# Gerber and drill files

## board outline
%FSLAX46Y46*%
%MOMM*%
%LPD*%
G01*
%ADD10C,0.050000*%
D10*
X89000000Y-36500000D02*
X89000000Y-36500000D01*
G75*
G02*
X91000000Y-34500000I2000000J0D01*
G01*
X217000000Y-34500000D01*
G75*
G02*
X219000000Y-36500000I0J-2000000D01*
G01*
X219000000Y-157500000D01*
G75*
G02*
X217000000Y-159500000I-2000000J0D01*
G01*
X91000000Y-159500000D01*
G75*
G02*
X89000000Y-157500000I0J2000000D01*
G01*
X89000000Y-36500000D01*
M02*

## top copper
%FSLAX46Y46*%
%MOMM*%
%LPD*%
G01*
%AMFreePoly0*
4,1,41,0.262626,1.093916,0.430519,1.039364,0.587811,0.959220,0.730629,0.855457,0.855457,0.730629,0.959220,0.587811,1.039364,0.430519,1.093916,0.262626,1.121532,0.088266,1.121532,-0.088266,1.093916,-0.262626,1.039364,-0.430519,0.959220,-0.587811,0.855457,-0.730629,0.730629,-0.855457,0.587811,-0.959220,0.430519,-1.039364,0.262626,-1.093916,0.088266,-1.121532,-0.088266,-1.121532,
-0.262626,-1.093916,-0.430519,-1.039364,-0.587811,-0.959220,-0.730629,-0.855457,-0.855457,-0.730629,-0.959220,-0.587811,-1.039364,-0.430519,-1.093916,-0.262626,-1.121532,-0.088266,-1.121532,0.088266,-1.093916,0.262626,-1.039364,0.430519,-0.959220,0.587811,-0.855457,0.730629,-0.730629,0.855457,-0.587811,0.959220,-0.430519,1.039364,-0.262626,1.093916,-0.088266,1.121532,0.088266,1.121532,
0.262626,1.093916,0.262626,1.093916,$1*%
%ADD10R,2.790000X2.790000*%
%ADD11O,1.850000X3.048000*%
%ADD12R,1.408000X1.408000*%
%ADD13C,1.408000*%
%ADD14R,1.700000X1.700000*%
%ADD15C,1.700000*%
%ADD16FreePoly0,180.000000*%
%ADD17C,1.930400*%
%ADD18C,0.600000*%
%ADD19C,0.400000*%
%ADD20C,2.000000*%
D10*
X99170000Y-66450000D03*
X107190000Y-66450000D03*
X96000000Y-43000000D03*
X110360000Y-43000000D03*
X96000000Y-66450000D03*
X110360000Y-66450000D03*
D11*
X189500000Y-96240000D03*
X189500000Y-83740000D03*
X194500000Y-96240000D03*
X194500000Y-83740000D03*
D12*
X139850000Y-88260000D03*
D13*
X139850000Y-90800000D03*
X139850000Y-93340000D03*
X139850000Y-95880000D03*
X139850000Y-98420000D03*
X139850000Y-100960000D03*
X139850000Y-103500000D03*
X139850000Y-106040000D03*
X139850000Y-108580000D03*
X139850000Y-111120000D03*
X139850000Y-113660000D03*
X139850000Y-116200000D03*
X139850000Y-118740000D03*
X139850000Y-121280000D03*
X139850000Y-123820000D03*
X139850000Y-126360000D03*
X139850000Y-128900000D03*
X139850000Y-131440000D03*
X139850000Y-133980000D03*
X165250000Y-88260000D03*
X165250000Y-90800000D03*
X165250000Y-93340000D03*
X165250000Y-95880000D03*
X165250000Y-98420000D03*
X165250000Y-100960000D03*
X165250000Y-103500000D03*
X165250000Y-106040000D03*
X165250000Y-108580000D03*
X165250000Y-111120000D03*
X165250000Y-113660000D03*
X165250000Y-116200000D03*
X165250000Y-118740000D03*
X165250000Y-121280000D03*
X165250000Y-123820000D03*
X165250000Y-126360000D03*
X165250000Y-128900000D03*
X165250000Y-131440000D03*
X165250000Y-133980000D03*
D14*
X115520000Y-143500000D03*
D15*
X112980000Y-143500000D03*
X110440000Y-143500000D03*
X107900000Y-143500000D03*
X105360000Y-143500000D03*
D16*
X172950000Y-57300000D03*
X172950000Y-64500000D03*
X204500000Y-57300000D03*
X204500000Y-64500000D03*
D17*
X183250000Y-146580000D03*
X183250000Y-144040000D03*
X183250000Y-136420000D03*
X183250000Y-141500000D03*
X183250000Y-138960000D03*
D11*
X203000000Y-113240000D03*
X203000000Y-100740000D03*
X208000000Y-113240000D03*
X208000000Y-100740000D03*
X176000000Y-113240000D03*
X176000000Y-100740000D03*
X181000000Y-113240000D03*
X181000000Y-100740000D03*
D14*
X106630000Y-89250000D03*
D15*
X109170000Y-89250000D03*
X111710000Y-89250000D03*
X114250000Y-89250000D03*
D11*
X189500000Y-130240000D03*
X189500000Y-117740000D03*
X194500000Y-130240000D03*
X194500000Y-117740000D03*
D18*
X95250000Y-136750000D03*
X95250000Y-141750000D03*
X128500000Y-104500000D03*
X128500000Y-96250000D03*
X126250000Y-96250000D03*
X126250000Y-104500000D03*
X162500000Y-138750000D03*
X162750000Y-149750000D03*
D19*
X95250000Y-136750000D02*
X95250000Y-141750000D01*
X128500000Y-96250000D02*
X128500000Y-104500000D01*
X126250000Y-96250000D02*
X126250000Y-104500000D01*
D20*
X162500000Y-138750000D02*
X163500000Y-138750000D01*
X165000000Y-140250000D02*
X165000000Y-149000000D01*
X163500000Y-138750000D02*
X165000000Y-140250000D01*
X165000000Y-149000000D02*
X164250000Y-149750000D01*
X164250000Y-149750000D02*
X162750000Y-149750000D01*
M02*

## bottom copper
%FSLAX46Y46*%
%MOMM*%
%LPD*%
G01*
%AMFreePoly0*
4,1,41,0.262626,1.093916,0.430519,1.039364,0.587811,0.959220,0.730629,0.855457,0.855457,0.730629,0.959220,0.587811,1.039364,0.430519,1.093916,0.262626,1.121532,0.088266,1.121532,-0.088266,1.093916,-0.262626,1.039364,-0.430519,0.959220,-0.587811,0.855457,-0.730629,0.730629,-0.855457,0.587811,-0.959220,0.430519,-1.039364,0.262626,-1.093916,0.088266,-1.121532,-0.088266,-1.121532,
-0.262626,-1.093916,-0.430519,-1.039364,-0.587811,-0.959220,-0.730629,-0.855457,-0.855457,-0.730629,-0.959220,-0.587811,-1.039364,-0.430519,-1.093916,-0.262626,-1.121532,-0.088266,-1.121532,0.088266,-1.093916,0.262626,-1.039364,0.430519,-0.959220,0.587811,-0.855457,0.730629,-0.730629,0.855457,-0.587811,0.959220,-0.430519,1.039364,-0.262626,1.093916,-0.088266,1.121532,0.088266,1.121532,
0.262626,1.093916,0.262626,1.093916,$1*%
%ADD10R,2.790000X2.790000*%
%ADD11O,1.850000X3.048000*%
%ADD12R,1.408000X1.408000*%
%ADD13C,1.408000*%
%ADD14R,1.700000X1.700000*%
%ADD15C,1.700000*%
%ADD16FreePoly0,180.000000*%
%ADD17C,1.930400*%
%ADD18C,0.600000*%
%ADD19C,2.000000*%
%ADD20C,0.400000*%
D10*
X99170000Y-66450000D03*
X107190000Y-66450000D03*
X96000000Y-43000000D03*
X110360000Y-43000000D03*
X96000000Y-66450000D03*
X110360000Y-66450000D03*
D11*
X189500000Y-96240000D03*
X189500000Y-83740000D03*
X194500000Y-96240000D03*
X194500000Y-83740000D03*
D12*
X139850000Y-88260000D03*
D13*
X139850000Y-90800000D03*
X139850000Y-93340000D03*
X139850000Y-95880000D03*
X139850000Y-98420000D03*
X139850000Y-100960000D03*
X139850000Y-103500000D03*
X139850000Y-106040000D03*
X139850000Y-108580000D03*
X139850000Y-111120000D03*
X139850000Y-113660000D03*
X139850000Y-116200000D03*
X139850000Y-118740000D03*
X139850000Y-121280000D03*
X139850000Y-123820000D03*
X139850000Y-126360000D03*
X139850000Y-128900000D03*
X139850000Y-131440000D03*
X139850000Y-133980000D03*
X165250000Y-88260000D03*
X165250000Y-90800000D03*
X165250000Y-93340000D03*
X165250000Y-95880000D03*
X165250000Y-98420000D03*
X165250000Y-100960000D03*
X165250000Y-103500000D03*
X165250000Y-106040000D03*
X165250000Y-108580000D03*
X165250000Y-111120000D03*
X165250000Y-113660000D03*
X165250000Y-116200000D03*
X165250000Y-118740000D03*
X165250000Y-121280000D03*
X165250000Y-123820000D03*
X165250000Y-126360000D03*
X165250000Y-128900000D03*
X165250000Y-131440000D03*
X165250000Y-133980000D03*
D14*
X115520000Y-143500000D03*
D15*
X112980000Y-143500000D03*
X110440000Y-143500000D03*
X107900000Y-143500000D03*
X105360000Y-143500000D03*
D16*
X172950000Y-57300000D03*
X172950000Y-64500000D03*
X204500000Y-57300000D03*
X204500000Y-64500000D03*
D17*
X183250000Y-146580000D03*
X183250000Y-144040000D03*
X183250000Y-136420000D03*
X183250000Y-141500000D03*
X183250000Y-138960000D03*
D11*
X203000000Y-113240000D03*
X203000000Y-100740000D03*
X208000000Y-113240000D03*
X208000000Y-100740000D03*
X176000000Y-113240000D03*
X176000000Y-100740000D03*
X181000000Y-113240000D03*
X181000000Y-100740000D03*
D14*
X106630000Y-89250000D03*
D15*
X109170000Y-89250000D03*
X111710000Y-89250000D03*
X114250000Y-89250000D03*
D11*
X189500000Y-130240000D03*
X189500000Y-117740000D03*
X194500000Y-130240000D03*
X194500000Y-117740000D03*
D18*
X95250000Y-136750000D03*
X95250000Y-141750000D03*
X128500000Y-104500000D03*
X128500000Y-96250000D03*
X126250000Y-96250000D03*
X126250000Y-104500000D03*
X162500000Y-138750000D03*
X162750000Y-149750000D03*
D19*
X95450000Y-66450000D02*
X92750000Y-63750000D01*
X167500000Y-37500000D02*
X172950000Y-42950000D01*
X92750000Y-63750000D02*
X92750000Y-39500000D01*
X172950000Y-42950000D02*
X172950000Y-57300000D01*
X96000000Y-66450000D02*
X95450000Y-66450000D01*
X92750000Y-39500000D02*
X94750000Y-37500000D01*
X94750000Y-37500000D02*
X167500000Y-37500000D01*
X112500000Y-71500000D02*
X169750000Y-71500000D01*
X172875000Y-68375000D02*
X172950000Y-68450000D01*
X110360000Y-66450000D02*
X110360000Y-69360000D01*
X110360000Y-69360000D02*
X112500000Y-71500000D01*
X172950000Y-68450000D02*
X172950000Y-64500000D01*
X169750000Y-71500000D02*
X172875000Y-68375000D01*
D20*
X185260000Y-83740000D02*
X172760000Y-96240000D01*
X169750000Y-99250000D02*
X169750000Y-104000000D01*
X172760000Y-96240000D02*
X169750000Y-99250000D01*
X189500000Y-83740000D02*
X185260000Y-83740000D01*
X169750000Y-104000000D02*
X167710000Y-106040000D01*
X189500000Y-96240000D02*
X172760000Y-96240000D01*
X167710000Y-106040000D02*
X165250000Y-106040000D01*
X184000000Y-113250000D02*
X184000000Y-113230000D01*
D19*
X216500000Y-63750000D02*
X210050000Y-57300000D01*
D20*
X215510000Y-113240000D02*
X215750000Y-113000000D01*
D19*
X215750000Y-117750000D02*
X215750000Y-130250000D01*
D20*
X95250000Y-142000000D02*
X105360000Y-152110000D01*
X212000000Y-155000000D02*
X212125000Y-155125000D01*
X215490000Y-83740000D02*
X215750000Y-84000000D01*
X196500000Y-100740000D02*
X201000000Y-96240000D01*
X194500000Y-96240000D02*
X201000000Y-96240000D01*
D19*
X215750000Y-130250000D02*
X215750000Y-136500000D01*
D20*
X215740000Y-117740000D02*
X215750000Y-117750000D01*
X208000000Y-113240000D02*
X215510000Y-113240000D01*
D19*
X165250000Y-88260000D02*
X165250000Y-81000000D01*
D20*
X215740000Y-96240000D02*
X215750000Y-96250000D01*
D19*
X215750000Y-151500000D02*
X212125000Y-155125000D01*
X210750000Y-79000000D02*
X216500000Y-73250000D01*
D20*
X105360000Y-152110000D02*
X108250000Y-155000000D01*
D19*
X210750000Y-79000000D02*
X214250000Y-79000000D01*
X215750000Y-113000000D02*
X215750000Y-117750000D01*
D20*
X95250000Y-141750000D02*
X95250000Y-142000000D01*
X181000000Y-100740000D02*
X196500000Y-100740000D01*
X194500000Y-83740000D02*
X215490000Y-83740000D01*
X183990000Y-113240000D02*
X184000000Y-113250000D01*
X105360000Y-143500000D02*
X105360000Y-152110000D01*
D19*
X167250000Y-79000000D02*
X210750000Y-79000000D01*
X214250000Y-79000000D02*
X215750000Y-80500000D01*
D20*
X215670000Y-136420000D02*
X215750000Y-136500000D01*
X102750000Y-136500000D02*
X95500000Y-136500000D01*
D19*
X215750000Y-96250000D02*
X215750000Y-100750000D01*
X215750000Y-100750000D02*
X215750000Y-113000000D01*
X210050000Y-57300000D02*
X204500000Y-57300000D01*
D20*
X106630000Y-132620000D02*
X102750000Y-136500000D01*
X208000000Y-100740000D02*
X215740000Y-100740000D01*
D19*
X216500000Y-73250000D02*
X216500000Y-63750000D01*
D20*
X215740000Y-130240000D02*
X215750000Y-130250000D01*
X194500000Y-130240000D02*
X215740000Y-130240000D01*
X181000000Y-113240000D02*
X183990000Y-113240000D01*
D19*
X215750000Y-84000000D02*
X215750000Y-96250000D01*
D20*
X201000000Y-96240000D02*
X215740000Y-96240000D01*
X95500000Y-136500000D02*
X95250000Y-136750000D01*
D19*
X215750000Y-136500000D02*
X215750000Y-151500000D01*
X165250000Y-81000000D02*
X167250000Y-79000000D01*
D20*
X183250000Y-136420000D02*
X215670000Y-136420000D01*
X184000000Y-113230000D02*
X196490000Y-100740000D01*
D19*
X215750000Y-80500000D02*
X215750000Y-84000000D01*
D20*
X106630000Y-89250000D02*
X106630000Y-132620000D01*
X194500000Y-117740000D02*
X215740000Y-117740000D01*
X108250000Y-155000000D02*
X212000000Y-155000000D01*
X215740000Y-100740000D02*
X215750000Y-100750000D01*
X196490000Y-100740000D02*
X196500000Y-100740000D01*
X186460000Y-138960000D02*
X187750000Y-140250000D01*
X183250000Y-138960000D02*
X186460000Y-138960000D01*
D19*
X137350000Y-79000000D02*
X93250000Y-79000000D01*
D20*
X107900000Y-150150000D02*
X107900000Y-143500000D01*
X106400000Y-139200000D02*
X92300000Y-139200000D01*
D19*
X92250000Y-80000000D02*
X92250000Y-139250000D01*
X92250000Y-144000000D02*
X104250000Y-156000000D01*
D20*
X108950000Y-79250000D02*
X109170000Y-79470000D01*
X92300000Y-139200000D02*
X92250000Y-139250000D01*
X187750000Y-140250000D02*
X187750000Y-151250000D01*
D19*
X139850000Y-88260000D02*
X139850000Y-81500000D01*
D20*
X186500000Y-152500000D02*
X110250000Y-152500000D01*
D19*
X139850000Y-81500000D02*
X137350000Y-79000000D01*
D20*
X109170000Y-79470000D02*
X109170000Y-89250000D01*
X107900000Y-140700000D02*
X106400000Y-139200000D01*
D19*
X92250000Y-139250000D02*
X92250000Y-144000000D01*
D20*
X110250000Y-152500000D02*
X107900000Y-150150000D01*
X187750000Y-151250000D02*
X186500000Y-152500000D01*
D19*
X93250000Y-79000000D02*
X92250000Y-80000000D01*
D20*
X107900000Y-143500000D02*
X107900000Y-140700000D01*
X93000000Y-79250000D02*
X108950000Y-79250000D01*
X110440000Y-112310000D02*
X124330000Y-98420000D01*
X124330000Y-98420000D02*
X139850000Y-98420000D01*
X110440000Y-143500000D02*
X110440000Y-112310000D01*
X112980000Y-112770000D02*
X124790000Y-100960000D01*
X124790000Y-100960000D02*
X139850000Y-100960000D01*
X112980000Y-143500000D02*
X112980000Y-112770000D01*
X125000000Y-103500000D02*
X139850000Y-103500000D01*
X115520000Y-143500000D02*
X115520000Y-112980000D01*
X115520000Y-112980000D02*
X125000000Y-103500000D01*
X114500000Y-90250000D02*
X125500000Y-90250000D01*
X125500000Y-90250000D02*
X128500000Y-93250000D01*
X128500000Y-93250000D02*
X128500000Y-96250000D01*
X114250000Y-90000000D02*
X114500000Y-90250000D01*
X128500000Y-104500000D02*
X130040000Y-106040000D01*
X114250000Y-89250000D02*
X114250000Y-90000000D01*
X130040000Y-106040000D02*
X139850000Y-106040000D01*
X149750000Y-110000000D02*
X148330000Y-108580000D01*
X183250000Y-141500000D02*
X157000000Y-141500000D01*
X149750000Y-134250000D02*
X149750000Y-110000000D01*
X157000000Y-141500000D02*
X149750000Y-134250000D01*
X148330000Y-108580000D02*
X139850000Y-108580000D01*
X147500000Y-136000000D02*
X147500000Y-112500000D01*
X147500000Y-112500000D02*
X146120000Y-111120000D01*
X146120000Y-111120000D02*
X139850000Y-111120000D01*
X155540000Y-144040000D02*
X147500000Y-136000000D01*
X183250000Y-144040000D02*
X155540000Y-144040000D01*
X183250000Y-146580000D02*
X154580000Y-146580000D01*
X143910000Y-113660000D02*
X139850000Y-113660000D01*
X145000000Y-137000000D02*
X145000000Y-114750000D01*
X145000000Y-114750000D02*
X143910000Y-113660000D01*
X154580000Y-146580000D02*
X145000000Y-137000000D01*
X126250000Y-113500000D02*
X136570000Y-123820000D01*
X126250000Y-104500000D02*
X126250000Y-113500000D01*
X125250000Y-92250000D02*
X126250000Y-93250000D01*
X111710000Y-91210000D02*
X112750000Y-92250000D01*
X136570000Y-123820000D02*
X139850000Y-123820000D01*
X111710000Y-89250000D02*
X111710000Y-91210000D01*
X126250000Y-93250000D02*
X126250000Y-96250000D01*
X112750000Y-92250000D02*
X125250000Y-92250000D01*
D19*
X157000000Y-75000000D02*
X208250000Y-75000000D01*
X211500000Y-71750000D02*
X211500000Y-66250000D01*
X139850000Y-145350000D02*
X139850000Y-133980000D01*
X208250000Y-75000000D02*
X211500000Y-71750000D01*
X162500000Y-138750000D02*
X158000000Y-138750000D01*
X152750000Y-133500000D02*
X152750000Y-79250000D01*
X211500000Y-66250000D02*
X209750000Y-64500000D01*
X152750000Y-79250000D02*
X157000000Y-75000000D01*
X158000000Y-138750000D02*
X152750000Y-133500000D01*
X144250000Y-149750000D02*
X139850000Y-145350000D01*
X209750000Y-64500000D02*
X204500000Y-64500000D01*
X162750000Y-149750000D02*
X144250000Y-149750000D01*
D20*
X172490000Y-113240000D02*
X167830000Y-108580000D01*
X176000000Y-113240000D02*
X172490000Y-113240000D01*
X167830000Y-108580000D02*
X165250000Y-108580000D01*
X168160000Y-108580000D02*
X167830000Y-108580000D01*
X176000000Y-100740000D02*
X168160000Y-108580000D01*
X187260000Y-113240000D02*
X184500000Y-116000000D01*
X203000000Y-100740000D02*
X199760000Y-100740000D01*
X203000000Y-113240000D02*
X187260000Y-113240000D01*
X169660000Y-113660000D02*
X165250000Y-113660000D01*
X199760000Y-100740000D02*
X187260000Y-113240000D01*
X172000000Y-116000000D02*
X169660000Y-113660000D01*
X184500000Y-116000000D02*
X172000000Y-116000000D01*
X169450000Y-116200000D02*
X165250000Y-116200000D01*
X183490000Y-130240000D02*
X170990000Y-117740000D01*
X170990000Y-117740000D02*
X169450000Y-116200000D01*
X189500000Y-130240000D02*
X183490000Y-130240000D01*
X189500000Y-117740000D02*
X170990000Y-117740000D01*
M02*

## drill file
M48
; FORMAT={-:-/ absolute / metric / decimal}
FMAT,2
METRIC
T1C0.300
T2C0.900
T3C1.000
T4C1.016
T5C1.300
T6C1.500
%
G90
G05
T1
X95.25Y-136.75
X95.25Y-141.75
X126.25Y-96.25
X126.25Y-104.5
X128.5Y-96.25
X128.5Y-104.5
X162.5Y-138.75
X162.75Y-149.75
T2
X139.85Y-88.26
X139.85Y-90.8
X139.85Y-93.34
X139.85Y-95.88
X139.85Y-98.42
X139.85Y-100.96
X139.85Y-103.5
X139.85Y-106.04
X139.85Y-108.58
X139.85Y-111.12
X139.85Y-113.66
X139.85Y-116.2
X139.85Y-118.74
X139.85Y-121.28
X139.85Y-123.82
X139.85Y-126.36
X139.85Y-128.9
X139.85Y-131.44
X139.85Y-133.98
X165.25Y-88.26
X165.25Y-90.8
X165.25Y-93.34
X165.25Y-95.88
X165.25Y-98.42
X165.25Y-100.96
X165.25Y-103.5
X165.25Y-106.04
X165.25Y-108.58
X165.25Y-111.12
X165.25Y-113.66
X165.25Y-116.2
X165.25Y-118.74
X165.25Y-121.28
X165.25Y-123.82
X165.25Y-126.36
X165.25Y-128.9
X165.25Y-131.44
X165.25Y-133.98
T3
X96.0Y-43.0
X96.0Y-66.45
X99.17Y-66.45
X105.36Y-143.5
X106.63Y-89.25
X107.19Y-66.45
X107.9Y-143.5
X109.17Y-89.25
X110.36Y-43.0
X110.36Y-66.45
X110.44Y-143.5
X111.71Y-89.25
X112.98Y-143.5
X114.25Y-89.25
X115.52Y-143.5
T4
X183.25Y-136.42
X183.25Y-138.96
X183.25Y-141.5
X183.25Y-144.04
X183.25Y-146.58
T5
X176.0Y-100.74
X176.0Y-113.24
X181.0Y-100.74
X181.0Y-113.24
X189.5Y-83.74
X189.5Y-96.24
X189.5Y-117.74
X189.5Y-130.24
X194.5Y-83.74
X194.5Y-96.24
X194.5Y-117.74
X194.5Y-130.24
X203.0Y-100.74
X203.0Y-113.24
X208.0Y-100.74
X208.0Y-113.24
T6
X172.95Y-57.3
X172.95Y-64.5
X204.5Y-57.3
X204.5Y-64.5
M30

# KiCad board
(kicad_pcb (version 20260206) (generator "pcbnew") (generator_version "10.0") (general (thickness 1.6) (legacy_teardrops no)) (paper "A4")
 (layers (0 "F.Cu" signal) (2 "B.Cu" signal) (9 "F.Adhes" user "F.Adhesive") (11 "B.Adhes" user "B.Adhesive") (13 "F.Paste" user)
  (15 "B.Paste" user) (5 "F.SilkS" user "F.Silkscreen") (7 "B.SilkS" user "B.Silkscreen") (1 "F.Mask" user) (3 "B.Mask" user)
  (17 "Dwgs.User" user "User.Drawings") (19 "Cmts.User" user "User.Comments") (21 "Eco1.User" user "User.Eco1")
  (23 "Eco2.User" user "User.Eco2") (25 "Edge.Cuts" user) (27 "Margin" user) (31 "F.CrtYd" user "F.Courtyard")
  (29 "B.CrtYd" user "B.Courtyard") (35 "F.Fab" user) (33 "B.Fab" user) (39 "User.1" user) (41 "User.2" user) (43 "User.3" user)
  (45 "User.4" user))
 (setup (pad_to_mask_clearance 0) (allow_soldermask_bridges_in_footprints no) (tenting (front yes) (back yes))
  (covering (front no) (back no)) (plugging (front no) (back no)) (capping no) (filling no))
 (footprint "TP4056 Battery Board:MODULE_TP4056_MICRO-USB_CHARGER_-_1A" (layer "F.Cu") (at 103.18 54.725 -90)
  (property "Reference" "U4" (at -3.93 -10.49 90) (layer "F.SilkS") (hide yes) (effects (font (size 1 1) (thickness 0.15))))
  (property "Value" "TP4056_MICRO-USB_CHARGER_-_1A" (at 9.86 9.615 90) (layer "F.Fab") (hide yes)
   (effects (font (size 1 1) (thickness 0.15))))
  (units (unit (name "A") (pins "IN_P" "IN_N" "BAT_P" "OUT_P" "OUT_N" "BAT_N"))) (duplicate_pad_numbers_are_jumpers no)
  (pad "BAT_N" thru_hole rect (at 11.725 4.01 270) (size 2.79 2.79) (drill 1) (layers "*.Cu" "*.Mask") (remove_unused_layers no)
   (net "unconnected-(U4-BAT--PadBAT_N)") (solder_mask_margin 0.102))
  (pad "BAT_P" thru_hole rect (at 11.725 -4.01 270) (size 2.79 2.79) (drill 1) (layers "*.Cu" "*.Mask") (remove_unused_layers no)
   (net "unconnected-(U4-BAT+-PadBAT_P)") (solder_mask_margin 0.102))
  (pad "IN_N" thru_hole rect (at -11.725 7.18 270) (size 2.79 2.79) (drill 1) (layers "*.Cu" "*.Mask") (remove_unused_layers no)
   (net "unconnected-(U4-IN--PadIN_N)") (solder_mask_margin 0.102))
  (pad "IN_P" thru_hole rect (at -11.725 -7.18 270) (size 2.79 2.79) (drill 1) (layers "*.Cu" "*.Mask") (remove_unused_layers no)
   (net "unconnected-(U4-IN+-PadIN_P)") (solder_mask_margin 0.102))
  (pad "OUT_N" thru_hole rect (at 11.725 7.18 270) (size 2.79 2.79) (drill 1) (layers "*.Cu" "*.Mask") (remove_unused_layers no)
   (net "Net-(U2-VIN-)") (solder_mask_margin 0.102))
  (pad "OUT_P" thru_hole rect (at 11.725 -7.18 270) (size 2.79 2.79) (drill 1) (layers "*.Cu" "*.Mask") (remove_unused_layers no)
   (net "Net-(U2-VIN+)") (solder_mask_margin 0.102)))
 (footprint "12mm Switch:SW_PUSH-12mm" (layer "F.Cu") (at 189.5 96.24 90)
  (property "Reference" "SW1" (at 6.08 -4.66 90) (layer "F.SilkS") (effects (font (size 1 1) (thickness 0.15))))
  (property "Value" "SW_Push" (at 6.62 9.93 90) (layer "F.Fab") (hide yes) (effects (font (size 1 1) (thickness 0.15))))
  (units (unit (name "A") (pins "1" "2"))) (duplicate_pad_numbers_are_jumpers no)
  (pad "1" thru_hole oval (at 0 0 90) (size 3.048 1.85) (drill 1.3) (layers "*.Cu" "*.Mask") (remove_unused_layers no) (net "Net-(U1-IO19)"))
  (pad "1" thru_hole oval (at 12.5 0 90) (size 3.048 1.85) (drill 1.3) (layers "*.Cu" "*.Mask") (remove_unused_layers no)
   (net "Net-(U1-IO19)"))
  (pad "2" thru_hole oval (at 0 5 90) (size 3.048 1.85) (drill 1.3) (layers "*.Cu" "*.Mask") (remove_unused_layers no) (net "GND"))
  (pad "2" thru_hole oval (at 12.5 5 90) (size 3.048 1.85) (drill 1.3) (layers "*.Cu" "*.Mask") (remove_unused_layers no) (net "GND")))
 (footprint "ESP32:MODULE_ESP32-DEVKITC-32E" (layer "F.Cu") (at 152.55 111.095)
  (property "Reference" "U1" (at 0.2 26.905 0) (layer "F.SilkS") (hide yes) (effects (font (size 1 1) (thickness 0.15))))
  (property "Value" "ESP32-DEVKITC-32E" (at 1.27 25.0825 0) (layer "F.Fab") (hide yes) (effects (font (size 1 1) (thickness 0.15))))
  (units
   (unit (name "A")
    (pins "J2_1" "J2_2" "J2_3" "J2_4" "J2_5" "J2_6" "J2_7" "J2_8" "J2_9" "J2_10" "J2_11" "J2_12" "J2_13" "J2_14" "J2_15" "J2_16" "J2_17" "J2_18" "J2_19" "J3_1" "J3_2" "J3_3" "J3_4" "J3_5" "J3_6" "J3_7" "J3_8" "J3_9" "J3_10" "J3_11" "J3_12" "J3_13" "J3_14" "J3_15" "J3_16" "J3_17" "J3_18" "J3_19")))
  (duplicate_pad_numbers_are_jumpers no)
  (pad "J2_1" thru_hole rect (at -12.7 -22.835) (size 1.408 1.408) (drill 0.9) (layers "*.Cu" "*.Mask") (remove_unused_layers no)
   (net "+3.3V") (solder_mask_margin 0.102))
  (pad "J2_2" thru_hole circle (at -12.7 -20.295) (size 1.408 1.408) (drill 0.9) (layers "*.Cu" "*.Mask") (remove_unused_layers no)
   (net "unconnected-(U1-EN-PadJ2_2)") (solder_mask_margin 0.102))
  (pad "J2_3" thru_hole circle (at -12.7 -17.755) (size 1.408 1.408) (drill 0.9) (layers "*.Cu" "*.Mask") (remove_unused_layers no)
   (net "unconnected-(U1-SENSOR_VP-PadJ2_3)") (solder_mask_margin 0.102))
  (pad "J2_4" thru_hole circle (at -12.7 -15.215) (size 1.408 1.408) (drill oval 0.9) (layers "*.Cu" "*.Mask") (remove_unused_layers no)
   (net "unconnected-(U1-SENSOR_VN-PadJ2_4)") (solder_mask_margin 0.102))
  (pad "J2_5" thru_hole circle (at -12.7 -12.675) (size 1.408 1.408) (drill 0.9) (layers "*.Cu" "*.Mask") (remove_unused_layers no)
   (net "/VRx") (solder_mask_margin 0.102))
  (pad "J2_6" thru_hole circle (at -12.7 -10.135) (size 1.408 1.408) (drill 0.9) (layers "*.Cu" "*.Mask") (remove_unused_layers no)
   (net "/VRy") (solder_mask_margin 0.102))
  (pad "J2_7" thru_hole circle (at -12.7 -7.595) (size 1.408 1.408) (drill 0.9) (layers "*.Cu" "*.Mask") (remove_unused_layers no)
   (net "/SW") (solder_mask_margin 0.102))
  (pad "J2_8" thru_hole circle (at -12.7 -5.055) (size 1.408 1.408) (drill 0.9) (layers "*.Cu" "*.Mask") (remove_unused_layers no)
   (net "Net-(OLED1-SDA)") (solder_mask_margin 0.102))
  (pad "J2_9" thru_hole circle (at -12.7 -2.515) (size 1.408 1.408) (drill 0.9) (layers "*.Cu" "*.Mask") (remove_unused_layers no)
   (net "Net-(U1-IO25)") (solder_mask_margin 0.102))
  (pad "J2_10" thru_hole circle (at -12.7 0.025) (size 1.408 1.408) (drill 0.9) (layers "*.Cu" "*.Mask") (remove_unused_layers no)
   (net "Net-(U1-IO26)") (solder_mask_margin 0.102))
  (pad "J2_11" thru_hole circle (at -12.7 2.565) (size 1.408 1.408) (drill 0.9) (layers "*.Cu" "*.Mask") (remove_unused_layers no)
   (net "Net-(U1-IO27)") (solder_mask_margin 0.102))
  (pad "J2_12" thru_hole circle (at -12.7 5.105) (size 1.408 1.408) (drill 0.9) (layers "*.Cu" "*.Mask") (remove_unused_layers no)
   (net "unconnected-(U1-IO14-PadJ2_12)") (solder_mask_margin 0.102))
  (pad "J2_13" thru_hole circle (at -12.7 7.645) (size 1.408 1.408) (drill 0.9) (layers "*.Cu" "*.Mask") (remove_unused_layers no)
   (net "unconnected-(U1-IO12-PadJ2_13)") (solder_mask_margin 0.102))
  (pad "J2_14" thru_hole circle (at -12.7 10.185) (size 1.408 1.408) (drill 0.9) (layers "*.Cu" "*.Mask") (remove_unused_layers no)
   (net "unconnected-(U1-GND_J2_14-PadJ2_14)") (solder_mask_margin 0.102))
  (pad "J2_15" thru_hole circle (at -12.7 12.725) (size 1.408 1.408) (drill 0.9) (layers "*.Cu" "*.Mask") (remove_unused_layers no)
   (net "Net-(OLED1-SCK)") (solder_mask_margin 0.102))
  (pad "J2_16" thru_hole circle (at -12.7 15.265) (size 1.408 1.408) (drill 0.9) (layers "*.Cu" "*.Mask") (remove_unused_layers no)
   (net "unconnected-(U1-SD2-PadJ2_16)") (solder_mask_margin 0.102))
  (pad "J2_17" thru_hole circle (at -12.7 17.805) (size 1.408 1.408) (drill 0.9) (layers "*.Cu" "*.Mask") (remove_unused_layers no)
   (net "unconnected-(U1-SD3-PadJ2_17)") (solder_mask_margin 0.102))
  (pad "J2_18" thru_hole circle (at -12.7 20.345) (size 1.408 1.408) (drill 0.9) (layers "*.Cu" "*.Mask") (remove_unused_layers no)
   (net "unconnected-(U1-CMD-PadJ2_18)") (solder_mask_margin 0.102))
  (pad "J2_19" thru_hole circle (at -12.7 22.885) (size 1.408 1.408) (drill 0.9) (layers "*.Cu" "*.Mask") (remove_unused_layers no)
   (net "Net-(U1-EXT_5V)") (solder_mask_margin 0.102))
  (pad "J3_1" thru_hole circle (at 12.7 -22.835) (size 1.408 1.408) (drill 0.9) (layers "*.Cu" "*.Mask") (remove_unused_layers no)
   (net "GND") (solder_mask_margin 0.102))
  (pad "J3_2" thru_hole circle (at 12.7 -20.295) (size 1.408 1.408) (drill 0.9) (layers "*.Cu" "*.Mask") (remove_unused_layers no)
   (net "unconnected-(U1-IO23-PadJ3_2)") (solder_mask_margin 0.102))
  (pad "J3_3" thru_hole circle (at 12.7 -17.755) (size 1.408 1.408) (drill 0.9) (layers "*.Cu" "*.Mask") (remove_unused_layers no)
   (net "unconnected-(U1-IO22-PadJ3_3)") (solder_mask_margin 0.102))
  (pad "J3_4" thru_hole circle (at 12.7 -15.215) (size 1.408 1.408) (drill 0.9) (layers "*.Cu" "*.Mask") (remove_unused_layers no)
   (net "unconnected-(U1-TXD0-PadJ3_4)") (solder_mask_margin 0.102))
  (pad "J3_5" thru_hole circle (at 12.7 -12.675) (size 1.408 1.408) (drill 0.9) (layers "*.Cu" "*.Mask") (remove_unused_layers no)
   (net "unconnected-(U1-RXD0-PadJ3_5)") (solder_mask_margin 0.102))
  (pad "J3_6" thru_hole circle (at 12.7 -10.135) (size 1.408 1.408) (drill 0.9) (layers "*.Cu" "*.Mask") (remove_unused_layers no)
   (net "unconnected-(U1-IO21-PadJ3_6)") (solder_mask_margin 0.102))
  (pad "J3_7" thru_hole circle (at 12.7 -7.595) (size 1.408 1.408) (drill 0.9) (layers "*.Cu" "*.Mask") (remove_unused_layers no)
   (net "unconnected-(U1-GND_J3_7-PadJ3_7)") (solder_mask_margin 0.102))
  (pad "J3_8" thru_hole circle (at 12.7 -5.055) (size 1.408 1.408) (drill 0.9) (layers "*.Cu" "*.Mask") (remove_unused_layers no)
   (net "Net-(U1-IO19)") (solder_mask_margin 0.102))
  (pad "J3_9" thru_hole circle (at 12.7 -2.515) (size 1.408 1.408) (drill 0.9) (layers "*.Cu" "*.Mask") (remove_unused_layers no)
   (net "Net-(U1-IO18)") (solder_mask_margin 0.102))
  (pad "J3_10" thru_hole circle (at 12.7 0.025) (size 1.408 1.408) (drill 0.9) (layers "*.Cu" "*.Mask") (remove_unused_layers no)
   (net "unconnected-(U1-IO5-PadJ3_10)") (solder_mask_margin 0.102))
  (pad "J3_11" thru_hole circle (at 12.7 2.565) (size 1.408 1.408) (drill 0.9) (layers "*.Cu" "*.Mask") (remove_unused_layers no)
   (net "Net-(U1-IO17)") (solder_mask_margin 0.102))
  (pad "J3_12" thru_hole circle (at 12.7 5.105) (size 1.408 1.408) (drill 0.9) (layers "*.Cu" "*.Mask") (remove_unused_layers no)
   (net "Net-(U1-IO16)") (solder_mask_margin 0.102))
  (pad "J3_13" thru_hole circle (at 12.7 7.645) (size 1.408 1.408) (drill 0.9) (layers "*.Cu" "*.Mask") (remove_unused_layers no)
   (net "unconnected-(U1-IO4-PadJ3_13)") (solder_mask_margin 0.102))
  (pad "J3_14" thru_hole circle (at 12.7 10.185) (size 1.408 1.408) (drill 0.9) (layers "*.Cu" "*.Mask") (remove_unused_layers no)
   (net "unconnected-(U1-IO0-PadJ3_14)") (solder_mask_margin 0.102))
  (pad "J3_15" thru_hole circle (at 12.7 12.725) (size 1.408 1.408) (drill 0.9) (layers "*.Cu" "*.Mask") (remove_unused_layers no)
   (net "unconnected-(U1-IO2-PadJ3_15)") (solder_mask_margin 0.102))
  (pad "J3_16" thru_hole circle (at 12.7 15.265) (size 1.408 1.408) (drill 0.9) (layers "*.Cu" "*.Mask") (remove_unused_layers no)
   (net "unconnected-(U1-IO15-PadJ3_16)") (solder_mask_margin 0.102))
  (pad "J3_17" thru_hole circle (at 12.7 17.805) (size 1.408 1.408) (drill 0.9) (layers "*.Cu" "*.Mask") (remove_unused_layers no)
   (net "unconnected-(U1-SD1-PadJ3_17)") (solder_mask_margin 0.102))
  (pad "J3_18" thru_hole circle (at 12.7 20.345) (size 1.408 1.408) (drill 0.9) (layers "*.Cu" "*.Mask") (remove_unused_layers no)
   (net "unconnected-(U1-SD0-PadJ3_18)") (solder_mask_margin 0.102))
  (pad "J3_19" thru_hole circle (at 12.7 22.885) (size 1.408 1.408) (drill 0.9) (layers "*.Cu" "*.Mask") (remove_unused_layers no)
   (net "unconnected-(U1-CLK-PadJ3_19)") (solder_mask_margin 0.102)))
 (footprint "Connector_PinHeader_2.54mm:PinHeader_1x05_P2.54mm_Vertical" (layer "F.Cu") (at 115.52 143.5 -90)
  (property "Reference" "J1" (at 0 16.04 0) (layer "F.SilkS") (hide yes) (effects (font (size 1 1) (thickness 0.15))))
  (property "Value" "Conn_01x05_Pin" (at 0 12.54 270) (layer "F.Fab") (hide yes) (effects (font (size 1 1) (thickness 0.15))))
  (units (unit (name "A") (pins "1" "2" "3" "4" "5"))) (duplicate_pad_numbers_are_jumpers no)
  (pad "1" thru_hole rect (at 0 0 270) (size 1.7 1.7) (drill 1) (layers "*.Cu" "*.Mask") (remove_unused_layers no) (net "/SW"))
  (pad "2" thru_hole circle (at 0 2.54 270) (size 1.7 1.7) (drill 1) (layers "*.Cu" "*.Mask") (remove_unused_layers no) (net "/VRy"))
  (pad "3" thru_hole circle (at 0 5.08 270) (size 1.7 1.7) (drill 1) (layers "*.Cu" "*.Mask") (remove_unused_layers no) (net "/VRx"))
  (pad "4" thru_hole circle (at 0 7.62 270) (size 1.7 1.7) (drill 1) (layers "*.Cu" "*.Mask") (remove_unused_layers no) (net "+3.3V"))
  (pad "5" thru_hole circle (at 0 10.16 270) (size 1.7 1.7) (drill 1) (layers "*.Cu" "*.Mask") (remove_unused_layers no) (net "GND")))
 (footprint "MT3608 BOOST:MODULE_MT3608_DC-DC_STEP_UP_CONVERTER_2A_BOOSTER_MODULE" (layer "F.Cu") (at 188.725 60.9 180)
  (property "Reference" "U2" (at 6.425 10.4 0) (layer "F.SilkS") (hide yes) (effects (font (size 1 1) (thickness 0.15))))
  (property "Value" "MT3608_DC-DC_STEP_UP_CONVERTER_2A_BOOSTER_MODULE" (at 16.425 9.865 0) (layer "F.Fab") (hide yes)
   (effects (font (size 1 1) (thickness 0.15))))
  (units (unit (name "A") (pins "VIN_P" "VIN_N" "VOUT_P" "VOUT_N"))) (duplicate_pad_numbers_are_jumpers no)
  (pad "VIN_N" thru_hole custom (at 15.775 3.6 180) (size 2.25 2.25) (drill 1.5) (layers "*.Cu") (remove_unused_layers no)
   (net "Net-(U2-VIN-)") (thermal_bridge_angle 90) (options (clearance outline) (anchor circle)) (primitives))
  (pad "VIN_P" thru_hole custom (at 15.775 -3.6 180) (size 2.25 2.25) (drill 1.5) (layers "*.Cu") (remove_unused_layers no)
   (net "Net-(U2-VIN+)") (thermal_bridge_angle 90) (options (clearance outline) (anchor circle)) (primitives))
  (pad "VOUT_N" thru_hole custom (at -15.775 3.6 180) (size 2.25 2.25) (drill 1.5) (layers "*.Cu") (remove_unused_layers no) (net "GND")
   (thermal_bridge_angle 90) (options (clearance outline) (anchor circle)) (primitives))
  (pad "VOUT_P" thru_hole custom (at -15.775 -3.6 180) (size 2.25 2.25) (drill 1.5) (layers "*.Cu") (remove_unused_layers no)
   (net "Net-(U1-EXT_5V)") (thermal_bridge_angle 90) (options (clearance outline) (anchor circle)) (primitives)))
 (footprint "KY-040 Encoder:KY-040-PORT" (layer "F.Cu") (at 183.25 140.23 90)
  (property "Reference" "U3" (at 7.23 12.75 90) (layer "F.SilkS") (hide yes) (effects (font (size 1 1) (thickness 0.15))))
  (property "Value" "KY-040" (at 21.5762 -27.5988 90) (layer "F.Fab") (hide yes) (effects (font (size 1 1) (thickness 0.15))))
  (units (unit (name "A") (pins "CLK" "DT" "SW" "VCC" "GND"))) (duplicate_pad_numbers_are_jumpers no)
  (pad "CLK" thru_hole circle (at -6.35 0 90) (size 1.9304 1.9304) (drill 1.016) (layers "*.Cu" "*.Mask") (remove_unused_layers no)
   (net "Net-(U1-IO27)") (solder_mask_margin 0.102))
  (pad "DT" thru_hole circle (at -3.81 0 90) (size 1.9304 1.9304) (drill 1.016) (layers "*.Cu" "*.Mask") (remove_unused_layers no)
   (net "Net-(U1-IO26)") (solder_mask_margin 0.102))
  (pad "GND" thru_hole circle (at 3.81 0 90) (size 1.9304 1.9304) (drill 1.016) (layers "*.Cu" "*.Mask") (remove_unused_layers no)
   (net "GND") (solder_mask_margin 0.102))
  (pad "SW" thru_hole circle (at -1.27 0 90) (size 1.9304 1.9304) (drill 1.016) (layers "*.Cu" "*.Mask") (remove_unused_layers no)
   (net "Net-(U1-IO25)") (solder_mask_margin 0.102))
  (pad "VCC" thru_hole circle (at 1.27 0 90) (size 1.9304 1.9304) (drill 1.016) (layers "*.Cu" "*.Mask") (remove_unused_layers no)
   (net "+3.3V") (solder_mask_margin 0.102)))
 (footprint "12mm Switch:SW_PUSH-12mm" (layer "F.Cu") (at 203 113.24 90)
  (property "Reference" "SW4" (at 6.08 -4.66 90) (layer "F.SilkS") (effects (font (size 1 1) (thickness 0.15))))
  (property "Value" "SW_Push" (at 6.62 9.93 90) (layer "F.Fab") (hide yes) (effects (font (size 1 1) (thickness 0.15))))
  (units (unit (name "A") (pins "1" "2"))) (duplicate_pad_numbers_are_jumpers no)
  (pad "1" thru_hole oval (at 0 0 90) (size 3.048 1.85) (drill 1.3) (layers "*.Cu" "*.Mask") (remove_unused_layers no) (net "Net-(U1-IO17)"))
  (pad "1" thru_hole oval (at 12.5 0 90) (size 3.048 1.85) (drill 1.3) (layers "*.Cu" "*.Mask") (remove_unused_layers no)
   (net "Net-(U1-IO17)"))
  (pad "2" thru_hole oval (at 0 5 90) (size 3.048 1.85) (drill 1.3) (layers "*.Cu" "*.Mask") (remove_unused_layers no) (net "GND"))
  (pad "2" thru_hole oval (at 12.5 5 90) (size 3.048 1.85) (drill 1.3) (layers "*.Cu" "*.Mask") (remove_unused_layers no) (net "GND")))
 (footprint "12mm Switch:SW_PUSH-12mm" (layer "F.Cu") (at 176 113.24 90)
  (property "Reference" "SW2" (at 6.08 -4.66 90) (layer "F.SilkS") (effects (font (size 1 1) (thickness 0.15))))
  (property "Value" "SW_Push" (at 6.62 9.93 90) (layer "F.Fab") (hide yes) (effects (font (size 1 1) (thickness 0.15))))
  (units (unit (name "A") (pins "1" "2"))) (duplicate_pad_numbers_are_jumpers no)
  (pad "1" thru_hole oval (at 0 0 90) (size 3.048 1.85) (drill 1.3) (layers "*.Cu" "*.Mask") (remove_unused_layers no) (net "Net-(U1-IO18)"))
  (pad "1" thru_hole oval (at 12.5 0 90) (size 3.048 1.85) (drill 1.3) (layers "*.Cu" "*.Mask") (remove_unused_layers no)
   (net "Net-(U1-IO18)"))
  (pad "2" thru_hole oval (at 0 5 90) (size 3.048 1.85) (drill 1.3) (layers "*.Cu" "*.Mask") (remove_unused_layers no) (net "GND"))
  (pad "2" thru_hole oval (at 12.5 5 90) (size 3.048 1.85) (drill 1.3) (layers "*.Cu" "*.Mask") (remove_unused_layers no) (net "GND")))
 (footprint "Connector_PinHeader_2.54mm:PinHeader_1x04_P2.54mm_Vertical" (layer "F.Cu") (at 106.63 89.25 90)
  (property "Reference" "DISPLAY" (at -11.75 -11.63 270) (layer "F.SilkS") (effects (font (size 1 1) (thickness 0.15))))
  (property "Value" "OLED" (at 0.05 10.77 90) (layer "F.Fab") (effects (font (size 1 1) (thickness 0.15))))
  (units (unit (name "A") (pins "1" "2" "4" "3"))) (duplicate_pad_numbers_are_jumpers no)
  (pad "1" thru_hole rect (at 0 0 90) (size 1.7 1.7) (drill 1) (layers "*.Cu" "*.Mask") (remove_unused_layers no) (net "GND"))
  (pad "2" thru_hole circle (at 0 2.54 90) (size 1.7 1.7) (drill 1) (layers "*.Cu" "*.Mask") (remove_unused_layers no) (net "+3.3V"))
  (pad "3" thru_hole circle (at 0 5.08 90) (size 1.7 1.7) (drill 1) (layers "*.Cu" "*.Mask") (remove_unused_layers no)
   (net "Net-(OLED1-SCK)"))
  (pad "4" thru_hole circle (at 0 7.62 90) (size 1.7 1.7) (drill 1) (layers "*.Cu" "*.Mask") (remove_unused_layers no)
   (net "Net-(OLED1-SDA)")))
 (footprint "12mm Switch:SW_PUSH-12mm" (layer "F.Cu") (at 189.5 130.24 90)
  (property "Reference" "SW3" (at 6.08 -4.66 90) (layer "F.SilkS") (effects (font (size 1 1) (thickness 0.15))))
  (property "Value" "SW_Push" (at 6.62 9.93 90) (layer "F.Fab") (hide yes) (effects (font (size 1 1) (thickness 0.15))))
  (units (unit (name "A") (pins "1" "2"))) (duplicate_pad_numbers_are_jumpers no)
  (pad "1" thru_hole oval (at 0 0 90) (size 3.048 1.85) (drill 1.3) (layers "*.Cu" "*.Mask") (remove_unused_layers no) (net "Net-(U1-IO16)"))
  (pad "1" thru_hole oval (at 12.5 0 90) (size 3.048 1.85) (drill 1.3) (layers "*.Cu" "*.Mask") (remove_unused_layers no)
   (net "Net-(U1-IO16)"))
  (pad "2" thru_hole oval (at 0 5 90) (size 3.048 1.85) (drill 1.3) (layers "*.Cu" "*.Mask") (remove_unused_layers no) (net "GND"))
  (pad "2" thru_hole oval (at 12.5 5 90) (size 3.048 1.85) (drill 1.3) (layers "*.Cu" "*.Mask") (remove_unused_layers no) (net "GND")))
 (gr_rect (start 89 34.5) (end 219 159.5) (radius 2) (stroke (width 0.05) (type solid)) (fill no) (layer "Edge.Cuts"))
 (segment (start 95.45 66.45) (end 92.75 63.75) (width 2) (layer "B.Cu") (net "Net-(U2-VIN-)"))
 (segment (start 167.5 37.5) (end 172.95 42.95) (width 2) (layer "B.Cu") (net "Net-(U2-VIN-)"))
 (segment (start 92.75 63.75) (end 92.75 39.5) (width 2) (layer "B.Cu") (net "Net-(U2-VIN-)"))
 (segment (start 172.95 42.95) (end 172.95 57.3) (width 2) (layer "B.Cu") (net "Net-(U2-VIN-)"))
 (segment (start 96 66.45) (end 95.45 66.45) (width 2) (layer "B.Cu") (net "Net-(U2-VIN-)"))
 (segment (start 92.75 39.5) (end 94.75 37.5) (width 2) (layer "B.Cu") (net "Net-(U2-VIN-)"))
 (segment (start 94.75 37.5) (end 167.5 37.5) (width 2) (layer "B.Cu") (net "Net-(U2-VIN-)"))
 (segment (start 112.5 71.5) (end 169.75 71.5) (width 2) (layer "B.Cu") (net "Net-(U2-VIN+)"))
 (segment (start 172.875 68.375) (end 172.95 68.45) (width 2) (layer "B.Cu") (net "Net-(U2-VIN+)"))
 (segment (start 110.36 66.45) (end 110.36 69.36) (width 2) (layer "B.Cu") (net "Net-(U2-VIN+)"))
 (segment (start 110.36 69.36) (end 112.5 71.5) (width 2) (layer "B.Cu") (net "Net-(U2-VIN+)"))
 (segment (start 172.95 68.45) (end 172.95 64.5) (width 2) (layer "B.Cu") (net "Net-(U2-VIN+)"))
 (segment (start 169.75 71.5) (end 172.875 68.375) (width 2) (layer "B.Cu") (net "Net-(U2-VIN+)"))
 (segment (start 185.26 83.74) (end 172.76 96.24) (width 0.4) (layer "B.Cu") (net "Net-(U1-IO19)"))
 (segment (start 169.75 99.25) (end 169.75 104) (width 0.4) (layer "B.Cu") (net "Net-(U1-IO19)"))
 (segment (start 172.76 96.24) (end 169.75 99.25) (width 0.4) (layer "B.Cu") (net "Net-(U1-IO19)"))
 (segment (start 189.5 83.74) (end 185.26 83.74) (width 0.4) (layer "B.Cu") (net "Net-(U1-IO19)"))
 (segment (start 169.75 104) (end 167.71 106.04) (width 0.4) (layer "B.Cu") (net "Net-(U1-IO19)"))
 (segment (start 189.5 96.24) (end 172.76 96.24) (width 0.4) (layer "B.Cu") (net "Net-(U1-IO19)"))
 (segment (start 167.71 106.04) (end 165.25 106.04) (width 0.4) (layer "B.Cu") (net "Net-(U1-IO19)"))
 (segment (start 95.25 136.75) (end 95.25 141.75) (width 0.4) (layer "F.Cu") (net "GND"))
 (via (at 95.25 136.75) (size 0.6) (drill 0.3) (layers "F.Cu" "B.Cu") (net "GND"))
 (via (at 95.25 141.75) (size 0.6) (drill 0.3) (layers "F.Cu" "B.Cu") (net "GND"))
 (segment (start 184 113.25) (end 184 113.23) (width 0.4) (layer "B.Cu") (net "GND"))
 (segment (start 216.5 63.75) (end 210.05 57.3) (width 2) (layer "B.Cu") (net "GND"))
 (segment (start 215.51 113.24) (end 215.75 113) (width 0.4) (layer "B.Cu") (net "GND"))
 (segment (start 215.75 117.75) (end 215.75 130.25) (width 2) (layer "B.Cu") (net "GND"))
 (segment (start 95.25 142) (end 105.36 152.11) (width 0.4) (layer "B.Cu") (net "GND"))
 (segment (start 212 155) (end 212.125 155.125) (width 0.4) (layer "B.Cu") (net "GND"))
 (segment (start 215.49 83.74) (end 215.75 84) (width 0.4) (layer "B.Cu") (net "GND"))
 (segment (start 196.5 100.74) (end 201 96.24) (width 0.4) (layer "B.Cu") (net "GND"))
 (segment (start 194.5 96.24) (end 201 96.24) (width 0.4) (layer "B.Cu") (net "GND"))
 (segment (start 215.75 130.25) (end 215.75 136.5) (width 2) (layer "B.Cu") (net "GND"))
 (segment (start 215.74 117.74) (end 215.75 117.75) (width 0.4) (layer "B.Cu") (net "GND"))
 (segment (start 208 113.24) (end 215.51 113.24) (width 0.4) (layer "B.Cu") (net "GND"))
 (segment (start 165.25 88.26) (end 165.25 81) (width 2) (layer "B.Cu") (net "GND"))
 (segment (start 215.74 96.24) (end 215.75 96.25) (width 0.4) (layer "B.Cu") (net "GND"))
 (segment (start 215.75 151.5) (end 212.125 155.125) (width 2) (layer "B.Cu") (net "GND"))
 (segment (start 210.75 79) (end 216.5 73.25) (width 2) (layer "B.Cu") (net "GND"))
 (segment (start 105.36 152.11) (end 108.25 155) (width 0.4) (layer "B.Cu") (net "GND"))
 (segment (start 210.75 79) (end 214.25 79) (width 2) (layer "B.Cu") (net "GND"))
 (segment (start 215.75 113) (end 215.75 117.75) (width 2) (layer "B.Cu") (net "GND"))
 (segment (start 95.25 141.75) (end 95.25 142) (width 0.4) (layer "B.Cu") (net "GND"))
 (segment (start 181 100.74) (end 196.5 100.74) (width 0.4) (layer "B.Cu") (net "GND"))
 (segment (start 194.5 83.74) (end 215.49 83.74) (width 0.4) (layer "B.Cu") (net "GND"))
 (segment (start 183.99 113.24) (end 184 113.25) (width 0.4) (layer "B.Cu") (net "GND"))
 (segment (start 105.36 143.5) (end 105.36 152.11) (width 0.4) (layer "B.Cu") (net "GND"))
 (segment (start 167.25 79) (end 210.75 79) (width 2) (layer "B.Cu") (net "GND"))
 (segment (start 214.25 79) (end 215.75 80.5) (width 2) (layer "B.Cu") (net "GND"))
 (segment (start 215.67 136.42) (end 215.75 136.5) (width 0.4) (layer "B.Cu") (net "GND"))
 (segment (start 102.75 136.5) (end 95.5 136.5) (width 0.4) (layer "B.Cu") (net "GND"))
 (segment (start 215.75 96.25) (end 215.75 100.75) (width 2) (layer "B.Cu") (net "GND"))
 (segment (start 215.75 100.75) (end 215.75 113) (width 2) (layer "B.Cu") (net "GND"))
 (segment (start 210.05 57.3) (end 204.5 57.3) (width 2) (layer "B.Cu") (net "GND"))
 (segment (start 106.63 132.62) (end 102.75 136.5) (width 0.4) (layer "B.Cu") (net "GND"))
 (segment (start 208 100.74) (end 215.74 100.74) (width 0.4) (layer "B.Cu") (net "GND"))
 (segment (start 216.5 73.25) (end 216.5 63.75) (width 2) (layer "B.Cu") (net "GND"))
 (segment (start 215.74 130.24) (end 215.75 130.25) (width 0.4) (layer "B.Cu") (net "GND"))
 (segment (start 194.5 130.24) (end 215.74 130.24) (width 0.4) (layer "B.Cu") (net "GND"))
 (segment (start 181 113.24) (end 183.99 113.24) (width 0.4) (layer "B.Cu") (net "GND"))
 (segment (start 215.75 84) (end 215.75 96.25) (width 2) (layer "B.Cu") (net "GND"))
 (segment (start 201 96.24) (end 215.74 96.24) (width 0.4) (layer "B.Cu") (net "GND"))
 (segment (start 95.5 136.5) (end 95.25 136.75) (width 0.4) (layer "B.Cu") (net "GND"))
 (segment (start 215.75 136.5) (end 215.75 151.5) (width 2) (layer "B.Cu") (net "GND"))
 (segment (start 165.25 81) (end 167.25 79) (width 2) (layer "B.Cu") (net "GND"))
 (segment (start 183.25 136.42) (end 215.67 136.42) (width 0.4) (layer "B.Cu") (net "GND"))
 (segment (start 184 113.23) (end 196.49 100.74) (width 0.4) (layer "B.Cu") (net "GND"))
 (segment (start 215.75 80.5) (end 215.75 84) (width 2) (layer "B.Cu") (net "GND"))
 (segment (start 106.63 89.25) (end 106.63 132.62) (width 0.4) (layer "B.Cu") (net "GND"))
 (segment (start 194.5 117.74) (end 215.74 117.74) (width 0.4) (layer "B.Cu") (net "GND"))
 (segment (start 108.25 155) (end 212 155) (width 0.4) (layer "B.Cu") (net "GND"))
 (segment (start 215.74 100.74) (end 215.75 100.75) (width 0.4) (layer "B.Cu") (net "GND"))
 (segment (start 196.49 100.74) (end 196.5 100.74) (width 0.4) (layer "B.Cu") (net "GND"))
 (segment (start 186.46 138.96) (end 187.75 140.25) (width 0.4) (layer "B.Cu") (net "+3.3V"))
 (segment (start 183.25 138.96) (end 186.46 138.96) (width 0.4) (layer "B.Cu") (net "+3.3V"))
 (segment (start 137.35 79) (end 93.25 79) (width 2) (layer "B.Cu") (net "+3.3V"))
 (segment (start 107.9 150.15) (end 107.9 143.5) (width 0.4) (layer "B.Cu") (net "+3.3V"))
 (segment (start 106.4 139.2) (end 92.3 139.2) (width 0.4) (layer "B.Cu") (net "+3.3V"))
 (segment (start 92.25 80) (end 92.25 139.25) (width 2) (layer "B.Cu") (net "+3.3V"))
 (segment (start 92.25 144) (end 104.25 156) (width 2) (layer "B.Cu") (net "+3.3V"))
 (segment (start 108.95 79.25) (end 109.17 79.47) (width 0.4) (layer "B.Cu") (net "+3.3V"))
 (segment (start 92.3 139.2) (end 92.25 139.25) (width 0.4) (layer "B.Cu") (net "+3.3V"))
 (segment (start 187.75 140.25) (end 187.75 151.25) (width 0.4) (layer "B.Cu") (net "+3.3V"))
 (segment (start 139.85 88.26) (end 139.85 81.5) (width 2) (layer "B.Cu") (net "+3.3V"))
 (segment (start 186.5 152.5) (end 110.25 152.5) (width 0.4) (layer "B.Cu") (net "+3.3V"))
 (segment (start 139.85 81.5) (end 137.35 79) (width 2) (layer "B.Cu") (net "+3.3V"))
 (segment (start 109.17 79.47) (end 109.17 89.25) (width 0.4) (layer "B.Cu") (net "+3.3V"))
 (segment (start 107.9 140.7) (end 106.4 139.2) (width 0.4) (layer "B.Cu") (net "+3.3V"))
 (segment (start 92.25 139.25) (end 92.25 144) (width 2) (layer "B.Cu") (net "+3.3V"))
 (segment (start 110.25 152.5) (end 107.9 150.15) (width 0.4) (layer "B.Cu") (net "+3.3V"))
 (segment (start 187.75 151.25) (end 186.5 152.5) (width 0.4) (layer "B.Cu") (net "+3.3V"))
 (segment (start 93.25 79) (end 92.25 80) (width 2) (layer "B.Cu") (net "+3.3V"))
 (segment (start 107.9 143.5) (end 107.9 140.7) (width 0.4) (layer "B.Cu") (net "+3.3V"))
 (segment (start 93 79.25) (end 108.95 79.25) (width 0.4) (layer "B.Cu") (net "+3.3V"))
 (segment (start 110.44 112.31) (end 124.33 98.42) (width 0.4) (layer "B.Cu") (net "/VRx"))
 (segment (start 124.33 98.42) (end 139.85 98.42) (width 0.4) (layer "B.Cu") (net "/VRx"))
 (segment (start 110.44 143.5) (end 110.44 112.31) (width 0.4) (layer "B.Cu") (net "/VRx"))
 (segment (start 112.98 112.77) (end 124.79 100.96) (width 0.4) (layer "B.Cu") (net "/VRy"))
 (segment (start 124.79 100.96) (end 139.85 100.96) (width 0.4) (layer "B.Cu") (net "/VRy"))
 (segment (start 112.98 143.5) (end 112.98 112.77) (width 0.4) (layer "B.Cu") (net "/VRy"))
 (segment (start 125 103.5) (end 139.85 103.5) (width 0.4) (layer "B.Cu") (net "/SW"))
 (segment (start 115.52 143.5) (end 115.52 112.98) (width 0.4) (layer "B.Cu") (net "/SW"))
 (segment (start 115.52 112.98) (end 125 103.5) (width 0.4) (layer "B.Cu") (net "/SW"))
 (segment (start 128.5 96.25) (end 128.5 104.5) (width 0.4) (layer "F.Cu") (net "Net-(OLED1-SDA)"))
 (via (at 128.5 104.5) (size 0.6) (drill 0.3) (layers "F.Cu" "B.Cu") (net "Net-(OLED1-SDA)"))
 (via (at 128.5 96.25) (size 0.6) (drill 0.3) (layers "F.Cu" "B.Cu") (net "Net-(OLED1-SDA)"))
 (segment (start 114.5 90.25) (end 125.5 90.25) (width 0.4) (layer "B.Cu") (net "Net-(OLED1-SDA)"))
 (segment (start 125.5 90.25) (end 128.5 93.25) (width 0.4) (layer "B.Cu") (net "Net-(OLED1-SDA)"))
 (segment (start 128.5 93.25) (end 128.5 96.25) (width 0.4) (layer "B.Cu") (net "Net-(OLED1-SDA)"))
 (segment (start 114.25 90) (end 114.5 90.25) (width 0.4) (layer "B.Cu") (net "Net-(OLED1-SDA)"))
 (segment (start 128.5 104.5) (end 130.04 106.04) (width 0.4) (layer "B.Cu") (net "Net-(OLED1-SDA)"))
 (segment (start 114.25 89.25) (end 114.25 90) (width 0.4) (layer "B.Cu") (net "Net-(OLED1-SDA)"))
 (segment (start 130.04 106.04) (end 139.85 106.04) (width 0.4) (layer "B.Cu") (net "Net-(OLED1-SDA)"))
 (segment (start 149.75 110) (end 148.33 108.58) (width 0.4) (layer "B.Cu") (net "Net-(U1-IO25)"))
 (segment (start 183.25 141.5) (end 157 141.5) (width 0.4) (layer "B.Cu") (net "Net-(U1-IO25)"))
 (segment (start 149.75 134.25) (end 149.75 110) (width 0.4) (layer "B.Cu") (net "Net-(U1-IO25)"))
 (segment (start 157 141.5) (end 149.75 134.25) (width 0.4) (layer "B.Cu") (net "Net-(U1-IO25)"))
 (segment (start 148.33 108.58) (end 139.85 108.58) (width 0.4) (layer "B.Cu") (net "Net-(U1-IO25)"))
 (segment (start 147.5 136) (end 147.5 112.5) (width 0.4) (layer "B.Cu") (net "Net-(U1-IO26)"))
 (segment (start 147.5 112.5) (end 146.12 111.12) (width 0.4) (layer "B.Cu") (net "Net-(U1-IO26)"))
 (segment (start 146.12 111.12) (end 139.85 111.12) (width 0.4) (layer "B.Cu") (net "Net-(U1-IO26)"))
 (segment (start 155.54 144.04) (end 147.5 136) (width 0.4) (layer "B.Cu") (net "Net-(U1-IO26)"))
 (segment (start 183.25 144.04) (end 155.54 144.04) (width 0.4) (layer "B.Cu") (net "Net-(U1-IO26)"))
 (segment (start 183.25 146.58) (end 154.58 146.58) (width 0.4) (layer "B.Cu") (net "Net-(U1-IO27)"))
 (segment (start 143.91 113.66) (end 139.85 113.66) (width 0.4) (layer "B.Cu") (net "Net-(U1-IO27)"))
 (segment (start 145 137) (end 145 114.75) (width 0.4) (layer "B.Cu") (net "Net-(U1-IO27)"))
 (segment (start 145 114.75) (end 143.91 113.66) (width 0.4) (layer "B.Cu") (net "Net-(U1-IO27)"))
 (segment (start 154.58 146.58) (end 145 137) (width 0.4) (layer "B.Cu") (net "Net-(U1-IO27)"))
 (segment (start 126.25 96.25) (end 126.25 104.5) (width 0.4) (layer "F.Cu") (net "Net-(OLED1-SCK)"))
 (via (at 126.25 96.25) (size 0.6) (drill 0.3) (layers "F.Cu" "B.Cu") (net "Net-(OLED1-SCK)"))
 (via (at 126.25 104.5) (size 0.6) (drill 0.3) (layers "F.Cu" "B.Cu") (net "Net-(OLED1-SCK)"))
 (segment (start 126.25 113.5) (end 136.57 123.82) (width 0.4) (layer "B.Cu") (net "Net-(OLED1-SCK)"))
 (segment (start 126.25 104.5) (end 126.25 113.5) (width 0.4) (layer "B.Cu") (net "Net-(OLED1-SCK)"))
 (segment (start 125.25 92.25) (end 126.25 93.25) (width 0.4) (layer "B.Cu") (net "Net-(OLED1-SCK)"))
 (segment (start 111.71 91.21) (end 112.75 92.25) (width 0.4) (layer "B.Cu") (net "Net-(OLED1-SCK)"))
 (segment (start 136.57 123.82) (end 139.85 123.82) (width 0.4) (layer "B.Cu") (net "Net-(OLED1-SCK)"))
 (segment (start 111.71 89.25) (end 111.71 91.21) (width 0.4) (layer "B.Cu") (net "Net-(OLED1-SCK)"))
 (segment (start 126.25 93.25) (end 126.25 96.25) (width 0.4) (layer "B.Cu") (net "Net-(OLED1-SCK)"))
 (segment (start 112.75 92.25) (end 125.25 92.25) (width 0.4) (layer "B.Cu") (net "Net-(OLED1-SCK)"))
 (segment (start 162.5 138.75) (end 163.5 138.75) (width 2) (layer "F.Cu") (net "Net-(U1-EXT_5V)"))
 (segment (start 165 140.25) (end 165 149) (width 2) (layer "F.Cu") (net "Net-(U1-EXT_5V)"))
 (segment (start 163.5 138.75) (end 165 140.25) (width 2) (layer "F.Cu") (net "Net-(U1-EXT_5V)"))
 (segment (start 165 149) (end 164.25 149.75) (width 2) (layer "F.Cu") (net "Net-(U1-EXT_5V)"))
 (segment (start 164.25 149.75) (end 162.75 149.75) (width 2) (layer "F.Cu") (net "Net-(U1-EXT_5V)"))
 (via (at 162.5 138.75) (size 0.6) (drill 0.3) (layers "F.Cu" "B.Cu") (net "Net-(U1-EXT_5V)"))
 (via (at 162.75 149.75) (size 0.6) (drill 0.3) (layers "F.Cu" "B.Cu") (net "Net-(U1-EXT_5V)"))
 (segment (start 157 75) (end 208.25 75) (width 2) (layer "B.Cu") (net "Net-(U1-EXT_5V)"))
 (segment (start 211.5 71.75) (end 211.5 66.25) (width 2) (layer "B.Cu") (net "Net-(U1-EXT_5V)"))
 (segment (start 139.85 145.35) (end 139.85 133.98) (width 2) (layer "B.Cu") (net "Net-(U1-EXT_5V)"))
 (segment (start 208.25 75) (end 211.5 71.75) (width 2) (layer "B.Cu") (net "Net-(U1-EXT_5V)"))
 (segment (start 162.5 138.75) (end 158 138.75) (width 2) (layer "B.Cu") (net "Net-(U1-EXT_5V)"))
 (segment (start 152.75 133.5) (end 152.75 79.25) (width 2) (layer "B.Cu") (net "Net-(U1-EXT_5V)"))
 (segment (start 211.5 66.25) (end 209.75 64.5) (width 2) (layer "B.Cu") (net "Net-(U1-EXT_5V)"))
 (segment (start 152.75 79.25) (end 157 75) (width 2) (layer "B.Cu") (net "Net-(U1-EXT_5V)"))
 (segment (start 158 138.75) (end 152.75 133.5) (width 2) (layer "B.Cu") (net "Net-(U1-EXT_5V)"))
 (segment (start 144.25 149.75) (end 139.85 145.35) (width 2) (layer "B.Cu") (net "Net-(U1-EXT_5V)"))
 (segment (start 209.75 64.5) (end 204.5 64.5) (width 2) (layer "B.Cu") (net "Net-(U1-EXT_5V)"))
 (segment (start 162.75 149.75) (end 144.25 149.75) (width 2) (layer "B.Cu") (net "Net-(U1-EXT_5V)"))
 (segment (start 172.49 113.24) (end 167.83 108.58) (width 0.4) (layer "B.Cu") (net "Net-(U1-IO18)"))
 (segment (start 176 113.24) (end 172.49 113.24) (width 0.4) (layer "B.Cu") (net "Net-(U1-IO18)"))
 (segment (start 167.83 108.58) (end 165.25 108.58) (width 0.4) (layer "B.Cu") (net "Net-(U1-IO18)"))
 (segment (start 168.16 108.58) (end 167.83 108.58) (width 0.4) (layer "B.Cu") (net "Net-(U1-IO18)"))
 (segment (start 176 100.74) (end 168.16 108.58) (width 0.4) (layer "B.Cu") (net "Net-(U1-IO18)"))
 (segment (start 187.26 113.24) (end 184.5 116) (width 0.4) (layer "B.Cu") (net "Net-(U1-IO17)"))
 (segment (start 203 100.74) (end 199.76 100.74) (width 0.4) (layer "B.Cu") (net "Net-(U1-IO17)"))
 (segment (start 203 113.24) (end 187.26 113.24) (width 0.4) (layer "B.Cu") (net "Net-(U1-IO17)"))
 (segment (start 169.66 113.66) (end 165.25 113.66) (width 0.4) (layer "B.Cu") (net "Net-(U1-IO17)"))
 (segment (start 199.76 100.74) (end 187.26 113.24) (width 0.4) (layer "B.Cu") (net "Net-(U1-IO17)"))
 (segment (start 172 116) (end 169.66 113.66) (width 0.4) (layer "B.Cu") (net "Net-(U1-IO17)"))
 (segment (start 184.5 116) (end 172 116) (width 0.4) (layer "B.Cu") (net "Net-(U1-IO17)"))
 (segment (start 169.45 116.2) (end 165.25 116.2) (width 0.4) (layer "B.Cu") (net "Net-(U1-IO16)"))
 (segment (start 183.49 130.24) (end 170.99 117.74) (width 0.4) (layer "B.Cu") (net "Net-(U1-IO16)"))
 (segment (start 170.99 117.74) (end 169.45 116.2) (width 0.4) (layer "B.Cu") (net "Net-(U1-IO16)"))
 (segment (start 189.5 130.24) (end 183.49 130.24) (width 0.4) (layer "B.Cu") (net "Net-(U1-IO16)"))
 (segment (start 189.5 117.74) (end 170.99 117.74) (width 0.4) (layer "B.Cu") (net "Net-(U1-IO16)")))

